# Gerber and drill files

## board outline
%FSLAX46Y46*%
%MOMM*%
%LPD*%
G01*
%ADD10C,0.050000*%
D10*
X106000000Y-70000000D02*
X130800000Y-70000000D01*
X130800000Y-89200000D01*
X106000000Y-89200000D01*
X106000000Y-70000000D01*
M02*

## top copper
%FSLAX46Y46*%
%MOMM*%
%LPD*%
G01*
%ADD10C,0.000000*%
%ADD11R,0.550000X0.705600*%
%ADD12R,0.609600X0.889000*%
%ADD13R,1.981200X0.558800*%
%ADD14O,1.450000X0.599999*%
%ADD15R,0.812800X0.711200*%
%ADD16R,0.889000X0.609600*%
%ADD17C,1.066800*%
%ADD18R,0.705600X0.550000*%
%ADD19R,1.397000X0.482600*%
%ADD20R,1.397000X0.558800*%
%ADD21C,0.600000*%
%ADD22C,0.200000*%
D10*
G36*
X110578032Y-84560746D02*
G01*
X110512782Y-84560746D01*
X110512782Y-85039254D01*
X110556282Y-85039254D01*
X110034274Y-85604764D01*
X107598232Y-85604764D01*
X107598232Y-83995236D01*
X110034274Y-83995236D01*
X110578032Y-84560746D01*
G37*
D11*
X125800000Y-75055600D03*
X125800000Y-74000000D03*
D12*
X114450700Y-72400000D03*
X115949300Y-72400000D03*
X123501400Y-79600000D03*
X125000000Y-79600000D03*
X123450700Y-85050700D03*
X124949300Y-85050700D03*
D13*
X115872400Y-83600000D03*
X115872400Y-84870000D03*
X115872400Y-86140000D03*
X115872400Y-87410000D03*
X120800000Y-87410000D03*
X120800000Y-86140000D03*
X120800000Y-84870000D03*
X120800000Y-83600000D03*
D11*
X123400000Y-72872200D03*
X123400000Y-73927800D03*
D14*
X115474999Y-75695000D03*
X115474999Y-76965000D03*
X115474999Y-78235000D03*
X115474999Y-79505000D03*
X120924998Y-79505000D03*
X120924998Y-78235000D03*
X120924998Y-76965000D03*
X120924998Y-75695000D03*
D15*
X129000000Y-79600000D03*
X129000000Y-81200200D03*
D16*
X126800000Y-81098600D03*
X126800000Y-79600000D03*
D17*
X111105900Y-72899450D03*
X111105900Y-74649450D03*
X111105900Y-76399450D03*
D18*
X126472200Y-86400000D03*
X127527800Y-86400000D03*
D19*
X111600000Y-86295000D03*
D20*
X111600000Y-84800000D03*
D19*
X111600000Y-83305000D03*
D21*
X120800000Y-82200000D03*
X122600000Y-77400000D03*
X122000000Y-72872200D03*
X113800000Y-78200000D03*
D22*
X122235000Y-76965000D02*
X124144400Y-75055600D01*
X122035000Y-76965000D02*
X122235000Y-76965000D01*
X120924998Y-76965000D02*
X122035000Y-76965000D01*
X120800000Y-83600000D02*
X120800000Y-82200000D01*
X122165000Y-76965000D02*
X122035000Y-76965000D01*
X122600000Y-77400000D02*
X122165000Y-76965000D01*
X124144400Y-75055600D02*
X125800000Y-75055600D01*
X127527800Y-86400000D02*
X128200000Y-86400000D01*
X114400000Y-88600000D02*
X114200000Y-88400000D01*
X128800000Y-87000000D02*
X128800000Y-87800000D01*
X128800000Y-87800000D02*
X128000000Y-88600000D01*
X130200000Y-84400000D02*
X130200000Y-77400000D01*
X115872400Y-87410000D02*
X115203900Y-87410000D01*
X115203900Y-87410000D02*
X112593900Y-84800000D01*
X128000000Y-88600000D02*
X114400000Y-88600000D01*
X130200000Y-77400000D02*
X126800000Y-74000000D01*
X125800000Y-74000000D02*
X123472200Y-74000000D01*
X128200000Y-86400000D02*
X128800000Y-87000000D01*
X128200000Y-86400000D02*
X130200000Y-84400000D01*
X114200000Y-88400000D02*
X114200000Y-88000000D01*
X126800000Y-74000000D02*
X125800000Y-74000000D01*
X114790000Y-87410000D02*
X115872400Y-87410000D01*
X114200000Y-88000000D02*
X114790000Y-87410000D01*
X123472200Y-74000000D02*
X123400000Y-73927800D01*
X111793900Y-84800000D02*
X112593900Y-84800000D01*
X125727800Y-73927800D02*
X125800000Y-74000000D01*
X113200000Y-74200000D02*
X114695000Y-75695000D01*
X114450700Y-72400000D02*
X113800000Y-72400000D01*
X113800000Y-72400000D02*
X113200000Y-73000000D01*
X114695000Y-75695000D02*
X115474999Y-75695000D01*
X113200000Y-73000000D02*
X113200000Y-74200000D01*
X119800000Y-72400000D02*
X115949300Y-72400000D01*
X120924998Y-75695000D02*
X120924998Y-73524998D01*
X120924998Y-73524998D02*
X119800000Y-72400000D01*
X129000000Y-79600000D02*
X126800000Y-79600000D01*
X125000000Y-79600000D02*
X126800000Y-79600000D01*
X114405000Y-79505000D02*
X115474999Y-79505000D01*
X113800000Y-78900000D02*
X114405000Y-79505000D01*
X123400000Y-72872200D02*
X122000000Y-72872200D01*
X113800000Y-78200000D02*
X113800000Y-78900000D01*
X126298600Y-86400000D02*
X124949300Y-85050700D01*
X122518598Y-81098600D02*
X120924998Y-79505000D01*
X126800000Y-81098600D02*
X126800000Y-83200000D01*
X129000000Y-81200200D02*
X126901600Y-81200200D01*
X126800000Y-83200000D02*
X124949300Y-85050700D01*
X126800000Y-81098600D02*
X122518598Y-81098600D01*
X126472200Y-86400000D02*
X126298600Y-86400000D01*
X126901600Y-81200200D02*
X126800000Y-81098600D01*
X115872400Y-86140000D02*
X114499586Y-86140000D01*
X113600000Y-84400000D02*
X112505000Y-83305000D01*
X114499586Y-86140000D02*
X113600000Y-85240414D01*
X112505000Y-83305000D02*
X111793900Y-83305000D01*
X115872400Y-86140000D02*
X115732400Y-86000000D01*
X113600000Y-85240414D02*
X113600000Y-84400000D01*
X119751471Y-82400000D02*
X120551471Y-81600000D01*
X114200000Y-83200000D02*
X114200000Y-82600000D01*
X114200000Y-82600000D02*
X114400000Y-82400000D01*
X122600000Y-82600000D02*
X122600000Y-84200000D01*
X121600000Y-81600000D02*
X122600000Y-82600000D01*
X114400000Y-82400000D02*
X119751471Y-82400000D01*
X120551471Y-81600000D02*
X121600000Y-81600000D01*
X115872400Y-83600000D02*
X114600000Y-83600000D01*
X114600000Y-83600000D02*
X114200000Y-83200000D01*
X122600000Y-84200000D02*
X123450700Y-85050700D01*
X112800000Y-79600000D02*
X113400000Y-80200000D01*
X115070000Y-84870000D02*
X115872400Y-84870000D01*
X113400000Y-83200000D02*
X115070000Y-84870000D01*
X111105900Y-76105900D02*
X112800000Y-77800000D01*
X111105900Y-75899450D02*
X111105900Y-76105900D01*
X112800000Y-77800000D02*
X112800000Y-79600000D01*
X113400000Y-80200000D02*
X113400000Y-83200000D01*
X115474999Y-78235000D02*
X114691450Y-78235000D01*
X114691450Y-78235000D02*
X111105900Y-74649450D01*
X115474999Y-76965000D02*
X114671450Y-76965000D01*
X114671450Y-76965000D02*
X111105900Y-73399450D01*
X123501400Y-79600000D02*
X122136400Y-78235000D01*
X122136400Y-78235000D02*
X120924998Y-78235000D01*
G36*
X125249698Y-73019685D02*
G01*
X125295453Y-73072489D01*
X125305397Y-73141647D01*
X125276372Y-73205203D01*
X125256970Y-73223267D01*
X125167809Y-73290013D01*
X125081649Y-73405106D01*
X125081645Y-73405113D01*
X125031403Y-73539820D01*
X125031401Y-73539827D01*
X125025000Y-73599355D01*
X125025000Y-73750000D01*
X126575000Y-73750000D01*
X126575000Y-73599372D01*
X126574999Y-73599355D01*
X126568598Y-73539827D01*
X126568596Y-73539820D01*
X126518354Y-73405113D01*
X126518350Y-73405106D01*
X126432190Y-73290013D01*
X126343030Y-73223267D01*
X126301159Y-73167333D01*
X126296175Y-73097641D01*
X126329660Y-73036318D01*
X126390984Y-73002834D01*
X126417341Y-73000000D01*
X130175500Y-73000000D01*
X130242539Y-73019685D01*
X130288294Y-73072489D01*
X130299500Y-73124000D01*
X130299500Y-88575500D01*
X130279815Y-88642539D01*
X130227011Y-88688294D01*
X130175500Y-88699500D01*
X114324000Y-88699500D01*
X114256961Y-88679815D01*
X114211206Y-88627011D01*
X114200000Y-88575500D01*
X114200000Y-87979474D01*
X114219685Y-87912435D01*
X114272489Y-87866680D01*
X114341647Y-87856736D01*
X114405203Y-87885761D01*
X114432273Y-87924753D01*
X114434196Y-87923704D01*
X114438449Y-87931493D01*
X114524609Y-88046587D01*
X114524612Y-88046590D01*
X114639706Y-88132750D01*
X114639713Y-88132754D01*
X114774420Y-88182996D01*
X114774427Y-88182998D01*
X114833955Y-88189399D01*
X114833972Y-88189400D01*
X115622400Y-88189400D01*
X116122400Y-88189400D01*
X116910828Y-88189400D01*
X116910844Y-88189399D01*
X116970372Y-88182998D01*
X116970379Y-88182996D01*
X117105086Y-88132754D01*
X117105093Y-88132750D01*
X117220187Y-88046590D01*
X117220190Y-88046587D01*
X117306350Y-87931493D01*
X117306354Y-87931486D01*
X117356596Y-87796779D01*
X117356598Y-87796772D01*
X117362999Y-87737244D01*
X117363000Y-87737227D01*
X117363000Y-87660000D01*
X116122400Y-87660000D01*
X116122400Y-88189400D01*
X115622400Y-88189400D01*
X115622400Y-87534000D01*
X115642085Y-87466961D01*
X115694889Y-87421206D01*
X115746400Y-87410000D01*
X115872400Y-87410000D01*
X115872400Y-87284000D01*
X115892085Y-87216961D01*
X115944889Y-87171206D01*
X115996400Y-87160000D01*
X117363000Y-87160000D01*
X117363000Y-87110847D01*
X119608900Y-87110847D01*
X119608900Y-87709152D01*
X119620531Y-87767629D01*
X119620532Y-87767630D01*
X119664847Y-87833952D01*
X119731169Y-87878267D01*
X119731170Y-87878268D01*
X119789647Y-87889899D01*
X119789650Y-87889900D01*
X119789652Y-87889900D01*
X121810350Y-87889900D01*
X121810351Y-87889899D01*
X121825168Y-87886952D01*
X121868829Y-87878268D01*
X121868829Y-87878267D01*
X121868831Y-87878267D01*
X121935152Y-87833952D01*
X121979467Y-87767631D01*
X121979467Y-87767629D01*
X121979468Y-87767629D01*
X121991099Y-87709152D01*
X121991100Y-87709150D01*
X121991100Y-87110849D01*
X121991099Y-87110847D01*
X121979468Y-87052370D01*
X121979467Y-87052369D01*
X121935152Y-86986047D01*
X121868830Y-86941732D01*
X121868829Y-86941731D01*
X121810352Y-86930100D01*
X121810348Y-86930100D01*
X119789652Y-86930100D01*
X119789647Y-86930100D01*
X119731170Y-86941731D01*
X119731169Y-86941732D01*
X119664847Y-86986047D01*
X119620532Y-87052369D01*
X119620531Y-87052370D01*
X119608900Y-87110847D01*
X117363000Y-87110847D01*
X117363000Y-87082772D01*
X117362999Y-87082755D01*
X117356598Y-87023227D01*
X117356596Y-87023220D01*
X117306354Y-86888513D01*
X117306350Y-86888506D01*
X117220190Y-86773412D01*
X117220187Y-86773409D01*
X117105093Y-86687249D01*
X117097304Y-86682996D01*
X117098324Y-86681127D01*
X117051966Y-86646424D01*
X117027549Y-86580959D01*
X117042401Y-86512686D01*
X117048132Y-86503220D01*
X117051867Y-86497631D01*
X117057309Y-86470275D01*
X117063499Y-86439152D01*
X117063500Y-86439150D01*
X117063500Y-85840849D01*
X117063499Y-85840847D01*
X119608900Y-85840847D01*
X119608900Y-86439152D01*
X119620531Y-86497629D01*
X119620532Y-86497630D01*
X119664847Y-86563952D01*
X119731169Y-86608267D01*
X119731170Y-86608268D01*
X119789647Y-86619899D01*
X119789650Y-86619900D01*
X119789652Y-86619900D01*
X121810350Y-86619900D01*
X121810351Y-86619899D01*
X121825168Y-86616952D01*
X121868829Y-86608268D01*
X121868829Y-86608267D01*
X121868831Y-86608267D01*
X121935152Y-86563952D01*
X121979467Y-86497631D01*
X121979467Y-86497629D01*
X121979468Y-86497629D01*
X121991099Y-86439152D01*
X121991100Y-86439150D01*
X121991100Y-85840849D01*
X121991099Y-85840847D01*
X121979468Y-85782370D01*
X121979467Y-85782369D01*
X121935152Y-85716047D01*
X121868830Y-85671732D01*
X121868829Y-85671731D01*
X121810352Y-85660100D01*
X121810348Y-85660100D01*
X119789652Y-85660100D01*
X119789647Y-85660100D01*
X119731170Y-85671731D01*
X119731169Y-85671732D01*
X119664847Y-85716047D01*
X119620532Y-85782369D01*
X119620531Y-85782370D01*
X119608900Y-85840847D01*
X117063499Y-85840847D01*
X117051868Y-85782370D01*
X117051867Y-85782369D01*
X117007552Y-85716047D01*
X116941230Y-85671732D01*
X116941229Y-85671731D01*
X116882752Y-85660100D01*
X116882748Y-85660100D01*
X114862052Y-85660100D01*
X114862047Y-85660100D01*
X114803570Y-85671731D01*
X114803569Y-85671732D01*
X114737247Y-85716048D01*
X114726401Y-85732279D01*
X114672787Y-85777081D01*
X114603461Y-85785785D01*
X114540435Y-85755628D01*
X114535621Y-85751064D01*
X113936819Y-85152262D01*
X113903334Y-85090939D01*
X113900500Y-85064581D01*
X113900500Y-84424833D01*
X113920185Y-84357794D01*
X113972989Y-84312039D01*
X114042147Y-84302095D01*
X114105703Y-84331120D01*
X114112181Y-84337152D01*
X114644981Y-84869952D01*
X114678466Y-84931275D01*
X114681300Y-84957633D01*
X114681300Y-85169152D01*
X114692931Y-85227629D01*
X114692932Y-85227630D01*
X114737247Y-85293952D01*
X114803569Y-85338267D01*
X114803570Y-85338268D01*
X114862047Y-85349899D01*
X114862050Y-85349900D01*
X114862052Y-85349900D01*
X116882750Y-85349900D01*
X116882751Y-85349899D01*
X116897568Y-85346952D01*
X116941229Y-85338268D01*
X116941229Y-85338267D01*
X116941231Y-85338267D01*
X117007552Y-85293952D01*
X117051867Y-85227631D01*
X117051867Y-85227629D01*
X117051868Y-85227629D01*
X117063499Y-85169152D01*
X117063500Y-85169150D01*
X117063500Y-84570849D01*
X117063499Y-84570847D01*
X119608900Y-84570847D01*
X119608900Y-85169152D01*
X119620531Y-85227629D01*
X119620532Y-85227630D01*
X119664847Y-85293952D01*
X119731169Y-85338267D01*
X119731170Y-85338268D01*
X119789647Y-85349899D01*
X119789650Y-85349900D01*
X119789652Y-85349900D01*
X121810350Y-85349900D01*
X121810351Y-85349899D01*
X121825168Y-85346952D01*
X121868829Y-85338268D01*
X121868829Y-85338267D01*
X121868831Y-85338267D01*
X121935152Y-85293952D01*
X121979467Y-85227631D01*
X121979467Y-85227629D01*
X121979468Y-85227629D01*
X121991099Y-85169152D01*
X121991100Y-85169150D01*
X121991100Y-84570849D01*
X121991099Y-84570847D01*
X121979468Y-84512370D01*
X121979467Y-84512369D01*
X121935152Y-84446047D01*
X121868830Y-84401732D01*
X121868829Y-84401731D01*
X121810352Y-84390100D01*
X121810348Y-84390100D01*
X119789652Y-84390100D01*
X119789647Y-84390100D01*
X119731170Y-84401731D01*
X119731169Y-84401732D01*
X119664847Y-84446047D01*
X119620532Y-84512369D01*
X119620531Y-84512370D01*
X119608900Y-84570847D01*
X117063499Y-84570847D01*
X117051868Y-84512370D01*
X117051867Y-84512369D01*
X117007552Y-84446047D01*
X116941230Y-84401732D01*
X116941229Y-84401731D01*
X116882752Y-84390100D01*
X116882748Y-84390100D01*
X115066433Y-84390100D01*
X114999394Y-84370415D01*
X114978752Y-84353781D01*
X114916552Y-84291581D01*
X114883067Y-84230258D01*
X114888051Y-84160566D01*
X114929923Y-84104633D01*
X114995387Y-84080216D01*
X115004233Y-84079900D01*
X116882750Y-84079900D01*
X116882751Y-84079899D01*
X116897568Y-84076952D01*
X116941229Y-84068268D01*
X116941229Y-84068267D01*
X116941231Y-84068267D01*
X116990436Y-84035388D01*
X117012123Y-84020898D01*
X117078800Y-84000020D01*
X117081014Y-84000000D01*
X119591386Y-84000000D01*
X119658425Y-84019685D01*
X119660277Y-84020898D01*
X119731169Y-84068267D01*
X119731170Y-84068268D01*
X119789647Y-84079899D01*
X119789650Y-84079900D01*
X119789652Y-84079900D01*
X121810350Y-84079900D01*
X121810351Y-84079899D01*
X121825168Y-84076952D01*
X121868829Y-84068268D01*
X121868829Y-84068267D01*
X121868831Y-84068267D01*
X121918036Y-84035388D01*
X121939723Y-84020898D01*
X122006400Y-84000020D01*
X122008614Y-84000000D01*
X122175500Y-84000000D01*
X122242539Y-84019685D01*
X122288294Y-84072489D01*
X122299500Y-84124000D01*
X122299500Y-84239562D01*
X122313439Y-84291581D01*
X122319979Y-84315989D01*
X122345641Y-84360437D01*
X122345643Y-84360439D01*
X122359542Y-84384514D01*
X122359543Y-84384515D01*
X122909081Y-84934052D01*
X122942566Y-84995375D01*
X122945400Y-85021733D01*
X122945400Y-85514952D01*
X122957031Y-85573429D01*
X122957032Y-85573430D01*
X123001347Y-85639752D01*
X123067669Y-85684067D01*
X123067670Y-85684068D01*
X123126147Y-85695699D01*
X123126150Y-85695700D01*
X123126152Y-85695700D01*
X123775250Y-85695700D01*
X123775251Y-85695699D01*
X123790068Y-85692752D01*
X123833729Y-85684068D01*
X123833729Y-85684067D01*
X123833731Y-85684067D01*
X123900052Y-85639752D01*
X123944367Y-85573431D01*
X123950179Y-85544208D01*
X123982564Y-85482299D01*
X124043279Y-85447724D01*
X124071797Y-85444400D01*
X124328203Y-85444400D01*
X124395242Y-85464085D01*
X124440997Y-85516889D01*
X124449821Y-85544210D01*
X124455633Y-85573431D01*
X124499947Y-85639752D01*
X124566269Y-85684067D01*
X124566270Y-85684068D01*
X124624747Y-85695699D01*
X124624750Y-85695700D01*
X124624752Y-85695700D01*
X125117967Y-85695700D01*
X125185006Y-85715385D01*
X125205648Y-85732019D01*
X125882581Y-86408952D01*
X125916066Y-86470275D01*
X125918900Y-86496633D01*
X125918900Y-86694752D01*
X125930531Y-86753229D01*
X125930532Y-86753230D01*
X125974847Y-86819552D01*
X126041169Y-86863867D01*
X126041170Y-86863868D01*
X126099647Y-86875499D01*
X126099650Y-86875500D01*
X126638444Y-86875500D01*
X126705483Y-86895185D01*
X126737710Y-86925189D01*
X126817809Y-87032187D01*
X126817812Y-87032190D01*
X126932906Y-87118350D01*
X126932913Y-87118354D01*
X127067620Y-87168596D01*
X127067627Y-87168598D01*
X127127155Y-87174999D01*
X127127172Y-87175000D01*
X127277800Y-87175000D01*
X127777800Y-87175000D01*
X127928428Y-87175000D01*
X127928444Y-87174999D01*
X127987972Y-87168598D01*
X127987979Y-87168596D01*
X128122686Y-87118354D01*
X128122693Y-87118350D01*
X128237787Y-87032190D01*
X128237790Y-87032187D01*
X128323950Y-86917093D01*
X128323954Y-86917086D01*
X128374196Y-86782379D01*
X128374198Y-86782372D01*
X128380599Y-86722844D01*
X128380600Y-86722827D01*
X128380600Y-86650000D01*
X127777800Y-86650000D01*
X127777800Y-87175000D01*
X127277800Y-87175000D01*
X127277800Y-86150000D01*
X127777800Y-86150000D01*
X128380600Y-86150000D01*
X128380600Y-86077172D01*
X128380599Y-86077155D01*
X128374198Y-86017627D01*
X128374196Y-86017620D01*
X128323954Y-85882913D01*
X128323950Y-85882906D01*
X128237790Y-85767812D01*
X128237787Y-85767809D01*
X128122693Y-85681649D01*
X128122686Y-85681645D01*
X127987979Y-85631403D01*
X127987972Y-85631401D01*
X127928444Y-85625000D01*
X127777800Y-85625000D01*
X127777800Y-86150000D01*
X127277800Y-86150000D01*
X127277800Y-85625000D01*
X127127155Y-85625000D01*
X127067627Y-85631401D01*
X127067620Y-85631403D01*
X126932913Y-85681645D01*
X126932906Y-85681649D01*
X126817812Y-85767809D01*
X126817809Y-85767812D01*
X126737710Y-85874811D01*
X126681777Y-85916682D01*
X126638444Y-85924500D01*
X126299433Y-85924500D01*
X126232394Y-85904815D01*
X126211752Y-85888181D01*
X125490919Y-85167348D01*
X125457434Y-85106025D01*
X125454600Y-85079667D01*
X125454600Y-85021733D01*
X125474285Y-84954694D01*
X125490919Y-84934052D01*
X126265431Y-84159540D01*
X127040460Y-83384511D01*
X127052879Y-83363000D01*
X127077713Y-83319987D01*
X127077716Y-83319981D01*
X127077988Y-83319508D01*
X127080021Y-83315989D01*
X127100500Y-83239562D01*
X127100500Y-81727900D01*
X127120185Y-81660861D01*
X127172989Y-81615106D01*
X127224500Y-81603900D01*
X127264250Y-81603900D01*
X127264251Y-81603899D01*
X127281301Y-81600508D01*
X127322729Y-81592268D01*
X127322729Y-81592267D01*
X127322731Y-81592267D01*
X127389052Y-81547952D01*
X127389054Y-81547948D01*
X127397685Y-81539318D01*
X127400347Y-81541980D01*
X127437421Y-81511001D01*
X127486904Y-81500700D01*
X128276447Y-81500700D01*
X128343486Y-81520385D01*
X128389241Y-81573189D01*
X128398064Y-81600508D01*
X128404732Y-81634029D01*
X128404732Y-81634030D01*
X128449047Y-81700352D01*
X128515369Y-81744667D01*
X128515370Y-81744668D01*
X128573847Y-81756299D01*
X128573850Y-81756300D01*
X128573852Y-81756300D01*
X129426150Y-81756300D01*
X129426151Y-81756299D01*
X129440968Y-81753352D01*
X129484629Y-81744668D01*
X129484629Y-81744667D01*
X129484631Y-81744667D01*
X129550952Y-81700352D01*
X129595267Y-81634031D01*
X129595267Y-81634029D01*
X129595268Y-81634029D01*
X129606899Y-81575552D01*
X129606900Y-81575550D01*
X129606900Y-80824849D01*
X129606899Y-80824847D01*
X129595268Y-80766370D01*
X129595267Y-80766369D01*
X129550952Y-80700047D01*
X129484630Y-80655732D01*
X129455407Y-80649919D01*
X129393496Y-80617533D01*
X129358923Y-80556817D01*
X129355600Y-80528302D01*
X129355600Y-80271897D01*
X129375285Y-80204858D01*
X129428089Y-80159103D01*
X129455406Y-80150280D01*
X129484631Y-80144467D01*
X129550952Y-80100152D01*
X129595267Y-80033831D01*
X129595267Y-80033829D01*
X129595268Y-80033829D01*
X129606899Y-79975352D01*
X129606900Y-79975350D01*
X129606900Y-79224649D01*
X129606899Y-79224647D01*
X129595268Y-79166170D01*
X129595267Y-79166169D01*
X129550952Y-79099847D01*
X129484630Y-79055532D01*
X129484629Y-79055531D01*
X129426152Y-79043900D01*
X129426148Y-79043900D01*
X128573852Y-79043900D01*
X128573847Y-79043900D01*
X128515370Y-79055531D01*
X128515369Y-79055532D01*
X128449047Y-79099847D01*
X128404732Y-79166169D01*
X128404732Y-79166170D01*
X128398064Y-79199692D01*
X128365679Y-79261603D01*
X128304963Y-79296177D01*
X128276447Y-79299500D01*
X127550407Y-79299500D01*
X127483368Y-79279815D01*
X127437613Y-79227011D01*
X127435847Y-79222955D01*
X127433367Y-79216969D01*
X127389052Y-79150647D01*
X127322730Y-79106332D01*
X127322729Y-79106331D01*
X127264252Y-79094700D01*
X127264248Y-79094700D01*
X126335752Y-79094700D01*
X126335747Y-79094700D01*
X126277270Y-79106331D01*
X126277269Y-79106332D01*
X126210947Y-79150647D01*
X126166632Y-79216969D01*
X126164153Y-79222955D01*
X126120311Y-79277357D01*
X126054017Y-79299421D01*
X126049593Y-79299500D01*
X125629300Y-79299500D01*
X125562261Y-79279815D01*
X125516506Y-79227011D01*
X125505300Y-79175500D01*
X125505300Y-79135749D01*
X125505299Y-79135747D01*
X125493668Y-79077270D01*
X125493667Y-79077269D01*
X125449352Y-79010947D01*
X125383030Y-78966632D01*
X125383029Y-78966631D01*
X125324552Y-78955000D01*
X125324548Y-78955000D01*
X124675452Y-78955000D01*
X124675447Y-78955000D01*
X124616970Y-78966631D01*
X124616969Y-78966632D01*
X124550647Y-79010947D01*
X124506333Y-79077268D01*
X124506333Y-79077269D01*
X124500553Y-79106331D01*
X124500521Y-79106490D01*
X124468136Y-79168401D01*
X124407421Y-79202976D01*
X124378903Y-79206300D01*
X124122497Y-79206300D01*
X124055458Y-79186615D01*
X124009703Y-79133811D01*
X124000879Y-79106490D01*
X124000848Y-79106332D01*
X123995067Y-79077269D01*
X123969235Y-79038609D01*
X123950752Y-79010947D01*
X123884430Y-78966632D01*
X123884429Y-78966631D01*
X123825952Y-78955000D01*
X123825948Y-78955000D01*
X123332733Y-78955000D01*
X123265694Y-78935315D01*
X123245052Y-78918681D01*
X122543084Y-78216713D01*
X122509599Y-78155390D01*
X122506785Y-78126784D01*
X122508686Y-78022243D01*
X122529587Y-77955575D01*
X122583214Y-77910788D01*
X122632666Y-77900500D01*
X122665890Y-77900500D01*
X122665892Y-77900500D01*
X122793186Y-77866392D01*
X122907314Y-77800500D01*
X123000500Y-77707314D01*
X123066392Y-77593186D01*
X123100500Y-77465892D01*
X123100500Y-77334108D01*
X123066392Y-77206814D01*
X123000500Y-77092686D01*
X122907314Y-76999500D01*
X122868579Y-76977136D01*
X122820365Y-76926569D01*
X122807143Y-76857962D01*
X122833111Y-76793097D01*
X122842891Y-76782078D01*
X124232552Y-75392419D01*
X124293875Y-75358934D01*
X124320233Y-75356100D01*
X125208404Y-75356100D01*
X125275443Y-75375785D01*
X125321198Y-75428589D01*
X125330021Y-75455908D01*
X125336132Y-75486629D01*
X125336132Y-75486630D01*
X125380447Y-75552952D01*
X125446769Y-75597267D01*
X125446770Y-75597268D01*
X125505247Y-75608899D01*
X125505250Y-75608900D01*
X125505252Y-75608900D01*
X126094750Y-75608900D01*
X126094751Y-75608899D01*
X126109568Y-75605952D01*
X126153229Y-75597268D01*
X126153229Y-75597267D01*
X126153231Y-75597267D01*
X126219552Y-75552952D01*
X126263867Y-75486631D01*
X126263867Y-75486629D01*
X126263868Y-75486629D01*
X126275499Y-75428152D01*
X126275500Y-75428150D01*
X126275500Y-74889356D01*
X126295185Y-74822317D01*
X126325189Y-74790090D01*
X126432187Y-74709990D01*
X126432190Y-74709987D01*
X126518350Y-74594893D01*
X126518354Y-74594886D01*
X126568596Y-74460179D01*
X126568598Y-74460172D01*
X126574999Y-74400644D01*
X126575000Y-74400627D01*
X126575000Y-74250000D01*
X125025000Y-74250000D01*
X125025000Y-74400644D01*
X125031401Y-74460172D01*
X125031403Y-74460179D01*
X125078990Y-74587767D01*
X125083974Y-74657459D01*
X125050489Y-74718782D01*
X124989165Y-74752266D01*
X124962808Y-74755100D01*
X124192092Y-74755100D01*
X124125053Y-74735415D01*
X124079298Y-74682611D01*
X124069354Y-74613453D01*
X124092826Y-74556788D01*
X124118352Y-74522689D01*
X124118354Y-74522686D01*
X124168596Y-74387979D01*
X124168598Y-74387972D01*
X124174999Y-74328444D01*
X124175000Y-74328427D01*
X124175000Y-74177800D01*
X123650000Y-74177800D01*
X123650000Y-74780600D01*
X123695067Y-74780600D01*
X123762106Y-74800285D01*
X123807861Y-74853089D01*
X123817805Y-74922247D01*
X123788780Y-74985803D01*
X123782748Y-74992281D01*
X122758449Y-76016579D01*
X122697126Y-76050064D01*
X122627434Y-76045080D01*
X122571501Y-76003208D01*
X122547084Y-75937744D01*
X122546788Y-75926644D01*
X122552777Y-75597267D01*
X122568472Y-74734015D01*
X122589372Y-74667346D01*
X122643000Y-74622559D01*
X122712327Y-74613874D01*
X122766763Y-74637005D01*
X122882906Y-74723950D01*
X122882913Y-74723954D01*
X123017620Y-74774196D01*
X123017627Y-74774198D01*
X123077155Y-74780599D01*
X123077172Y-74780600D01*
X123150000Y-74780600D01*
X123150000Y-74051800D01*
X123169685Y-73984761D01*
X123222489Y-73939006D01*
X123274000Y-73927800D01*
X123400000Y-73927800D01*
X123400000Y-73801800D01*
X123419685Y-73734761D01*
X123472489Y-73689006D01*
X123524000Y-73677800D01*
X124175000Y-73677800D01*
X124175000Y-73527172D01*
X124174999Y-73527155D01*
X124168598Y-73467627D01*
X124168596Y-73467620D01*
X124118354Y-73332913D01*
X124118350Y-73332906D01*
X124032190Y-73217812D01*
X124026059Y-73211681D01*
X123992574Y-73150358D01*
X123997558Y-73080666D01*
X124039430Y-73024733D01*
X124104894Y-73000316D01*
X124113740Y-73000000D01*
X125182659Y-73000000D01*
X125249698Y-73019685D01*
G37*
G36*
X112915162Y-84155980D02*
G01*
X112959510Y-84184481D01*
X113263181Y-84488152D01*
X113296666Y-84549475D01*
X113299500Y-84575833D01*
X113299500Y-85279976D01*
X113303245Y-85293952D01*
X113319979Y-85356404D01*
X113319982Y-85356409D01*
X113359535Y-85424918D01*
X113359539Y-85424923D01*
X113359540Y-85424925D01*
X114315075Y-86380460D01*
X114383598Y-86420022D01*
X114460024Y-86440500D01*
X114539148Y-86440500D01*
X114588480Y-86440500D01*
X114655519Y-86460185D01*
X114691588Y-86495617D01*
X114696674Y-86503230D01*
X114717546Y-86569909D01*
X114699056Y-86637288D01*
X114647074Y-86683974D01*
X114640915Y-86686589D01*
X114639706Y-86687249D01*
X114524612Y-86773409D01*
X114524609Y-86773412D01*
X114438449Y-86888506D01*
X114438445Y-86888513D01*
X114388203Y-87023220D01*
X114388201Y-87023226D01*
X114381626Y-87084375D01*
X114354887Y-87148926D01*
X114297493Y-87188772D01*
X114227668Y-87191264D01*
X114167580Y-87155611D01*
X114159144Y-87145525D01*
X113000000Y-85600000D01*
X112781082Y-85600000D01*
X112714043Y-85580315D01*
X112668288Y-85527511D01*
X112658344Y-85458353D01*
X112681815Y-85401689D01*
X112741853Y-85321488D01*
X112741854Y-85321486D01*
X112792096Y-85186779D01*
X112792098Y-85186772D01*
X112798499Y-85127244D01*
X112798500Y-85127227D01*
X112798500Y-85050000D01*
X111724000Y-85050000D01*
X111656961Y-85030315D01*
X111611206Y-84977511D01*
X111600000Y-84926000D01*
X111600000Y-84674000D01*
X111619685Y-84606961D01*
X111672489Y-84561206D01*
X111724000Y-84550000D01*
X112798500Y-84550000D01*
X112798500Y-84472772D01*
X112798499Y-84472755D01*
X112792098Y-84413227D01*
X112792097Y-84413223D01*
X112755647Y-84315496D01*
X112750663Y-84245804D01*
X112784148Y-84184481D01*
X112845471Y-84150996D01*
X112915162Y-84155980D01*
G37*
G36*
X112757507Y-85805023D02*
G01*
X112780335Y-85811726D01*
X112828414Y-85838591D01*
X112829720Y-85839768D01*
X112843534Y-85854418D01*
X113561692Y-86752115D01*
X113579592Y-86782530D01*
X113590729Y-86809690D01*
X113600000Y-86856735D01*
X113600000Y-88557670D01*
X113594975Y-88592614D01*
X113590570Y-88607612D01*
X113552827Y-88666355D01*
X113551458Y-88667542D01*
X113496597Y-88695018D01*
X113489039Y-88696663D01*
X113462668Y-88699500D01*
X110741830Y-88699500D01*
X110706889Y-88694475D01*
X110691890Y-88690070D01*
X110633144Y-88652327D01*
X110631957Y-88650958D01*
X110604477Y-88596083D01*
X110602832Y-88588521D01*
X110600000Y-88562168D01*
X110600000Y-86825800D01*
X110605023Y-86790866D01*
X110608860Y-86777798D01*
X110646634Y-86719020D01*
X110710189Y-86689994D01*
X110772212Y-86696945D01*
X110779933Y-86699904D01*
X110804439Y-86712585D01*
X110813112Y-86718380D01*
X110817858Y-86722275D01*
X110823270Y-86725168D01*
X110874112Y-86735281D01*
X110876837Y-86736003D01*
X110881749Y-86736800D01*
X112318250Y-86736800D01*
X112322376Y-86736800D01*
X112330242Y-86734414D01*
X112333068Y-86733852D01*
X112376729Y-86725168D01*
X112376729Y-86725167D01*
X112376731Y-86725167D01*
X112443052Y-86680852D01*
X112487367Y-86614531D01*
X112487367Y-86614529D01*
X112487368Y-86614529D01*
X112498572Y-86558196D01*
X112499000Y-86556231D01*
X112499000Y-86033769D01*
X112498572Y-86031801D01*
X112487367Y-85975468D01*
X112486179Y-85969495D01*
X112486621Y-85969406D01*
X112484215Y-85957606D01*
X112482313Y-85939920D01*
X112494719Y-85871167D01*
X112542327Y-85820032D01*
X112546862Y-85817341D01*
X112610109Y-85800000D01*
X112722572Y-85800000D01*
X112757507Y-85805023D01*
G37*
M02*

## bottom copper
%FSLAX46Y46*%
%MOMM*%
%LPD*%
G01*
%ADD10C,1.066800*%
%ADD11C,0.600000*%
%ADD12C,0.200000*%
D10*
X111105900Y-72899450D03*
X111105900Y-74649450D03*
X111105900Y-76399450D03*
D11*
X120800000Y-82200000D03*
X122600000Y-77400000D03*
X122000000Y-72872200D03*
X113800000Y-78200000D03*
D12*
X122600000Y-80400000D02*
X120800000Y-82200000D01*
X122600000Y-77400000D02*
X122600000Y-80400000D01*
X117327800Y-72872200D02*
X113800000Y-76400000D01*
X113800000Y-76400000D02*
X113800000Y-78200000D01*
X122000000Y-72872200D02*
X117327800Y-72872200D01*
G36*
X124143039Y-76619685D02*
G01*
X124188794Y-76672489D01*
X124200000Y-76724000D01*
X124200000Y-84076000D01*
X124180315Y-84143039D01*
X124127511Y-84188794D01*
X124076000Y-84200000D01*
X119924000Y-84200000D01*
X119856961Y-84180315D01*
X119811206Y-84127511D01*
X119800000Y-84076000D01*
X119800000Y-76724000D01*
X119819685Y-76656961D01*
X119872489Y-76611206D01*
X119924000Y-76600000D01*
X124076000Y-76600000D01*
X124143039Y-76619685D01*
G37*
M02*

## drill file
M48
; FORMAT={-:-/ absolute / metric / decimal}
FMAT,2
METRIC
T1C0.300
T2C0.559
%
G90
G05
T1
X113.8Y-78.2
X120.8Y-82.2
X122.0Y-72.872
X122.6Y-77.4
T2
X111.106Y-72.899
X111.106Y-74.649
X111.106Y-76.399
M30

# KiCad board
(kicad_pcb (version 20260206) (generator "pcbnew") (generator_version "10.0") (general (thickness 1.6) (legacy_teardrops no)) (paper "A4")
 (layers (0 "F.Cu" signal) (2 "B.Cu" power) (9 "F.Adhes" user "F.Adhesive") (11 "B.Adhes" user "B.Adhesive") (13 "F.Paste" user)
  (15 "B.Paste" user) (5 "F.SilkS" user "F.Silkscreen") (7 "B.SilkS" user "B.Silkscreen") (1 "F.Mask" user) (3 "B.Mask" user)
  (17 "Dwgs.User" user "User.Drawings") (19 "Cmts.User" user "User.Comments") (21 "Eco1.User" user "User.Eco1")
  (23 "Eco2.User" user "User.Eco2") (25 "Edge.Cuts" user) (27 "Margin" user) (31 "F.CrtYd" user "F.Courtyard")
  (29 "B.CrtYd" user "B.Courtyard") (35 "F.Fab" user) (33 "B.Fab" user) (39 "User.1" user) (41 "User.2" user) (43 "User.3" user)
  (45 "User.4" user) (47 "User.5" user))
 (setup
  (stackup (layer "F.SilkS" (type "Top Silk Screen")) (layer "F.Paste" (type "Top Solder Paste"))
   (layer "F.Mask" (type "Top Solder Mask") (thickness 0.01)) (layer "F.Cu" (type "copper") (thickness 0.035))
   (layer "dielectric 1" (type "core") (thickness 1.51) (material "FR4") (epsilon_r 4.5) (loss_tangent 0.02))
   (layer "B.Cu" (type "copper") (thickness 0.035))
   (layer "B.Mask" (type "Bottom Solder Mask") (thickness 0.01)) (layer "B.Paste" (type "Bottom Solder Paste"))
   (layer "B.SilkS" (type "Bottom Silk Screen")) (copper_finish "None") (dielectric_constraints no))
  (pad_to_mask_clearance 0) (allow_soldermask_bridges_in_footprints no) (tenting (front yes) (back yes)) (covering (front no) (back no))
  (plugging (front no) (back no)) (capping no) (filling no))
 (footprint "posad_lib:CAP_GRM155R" (layer "F.Cu") (at 125.8 74.5278 90)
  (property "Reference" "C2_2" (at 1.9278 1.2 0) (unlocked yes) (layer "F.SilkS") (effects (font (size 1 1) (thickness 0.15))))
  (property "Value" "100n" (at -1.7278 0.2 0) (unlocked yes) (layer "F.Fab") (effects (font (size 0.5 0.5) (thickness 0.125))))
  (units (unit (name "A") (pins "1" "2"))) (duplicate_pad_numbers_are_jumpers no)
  (pad "1" smd rect (at -0.5278 0 90) (size 0.7056 0.55) (layers "F.Cu" "F.Mask" "F.Paste") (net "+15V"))
  (pad "2" smd rect (at 0.5278 0 90) (size 0.7056 0.55) (layers "F.Cu" "F.Mask" "F.Paste") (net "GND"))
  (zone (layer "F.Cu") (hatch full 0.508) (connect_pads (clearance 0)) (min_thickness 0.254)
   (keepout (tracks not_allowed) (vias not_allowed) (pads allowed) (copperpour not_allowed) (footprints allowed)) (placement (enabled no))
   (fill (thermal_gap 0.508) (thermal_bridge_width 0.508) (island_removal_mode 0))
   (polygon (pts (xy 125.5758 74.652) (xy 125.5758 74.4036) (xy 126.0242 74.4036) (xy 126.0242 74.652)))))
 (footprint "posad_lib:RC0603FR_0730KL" (layer "F.Cu") (at 115.2 72.4)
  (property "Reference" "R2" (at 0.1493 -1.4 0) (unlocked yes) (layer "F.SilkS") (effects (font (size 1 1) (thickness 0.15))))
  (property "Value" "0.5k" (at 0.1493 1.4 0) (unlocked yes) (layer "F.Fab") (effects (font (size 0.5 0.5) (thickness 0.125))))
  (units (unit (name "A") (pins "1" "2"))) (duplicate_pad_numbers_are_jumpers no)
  (pad "1" smd rect (at -0.7493 0) (size 0.6096 0.889) (layers "F.Cu" "F.Mask" "F.Paste") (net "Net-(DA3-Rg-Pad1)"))
  (pad "2" smd rect (at 0.7493 0) (size 0.6096 0.889) (layers "F.Cu" "F.Mask" "F.Paste") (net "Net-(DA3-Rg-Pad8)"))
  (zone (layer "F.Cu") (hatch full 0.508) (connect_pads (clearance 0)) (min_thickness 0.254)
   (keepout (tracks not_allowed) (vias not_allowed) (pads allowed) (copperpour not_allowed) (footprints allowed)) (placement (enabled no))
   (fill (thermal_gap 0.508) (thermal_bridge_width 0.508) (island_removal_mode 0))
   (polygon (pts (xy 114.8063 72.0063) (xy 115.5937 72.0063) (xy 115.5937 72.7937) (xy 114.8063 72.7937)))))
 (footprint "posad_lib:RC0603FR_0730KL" (layer "F.Cu") (at 124.2507 79.6)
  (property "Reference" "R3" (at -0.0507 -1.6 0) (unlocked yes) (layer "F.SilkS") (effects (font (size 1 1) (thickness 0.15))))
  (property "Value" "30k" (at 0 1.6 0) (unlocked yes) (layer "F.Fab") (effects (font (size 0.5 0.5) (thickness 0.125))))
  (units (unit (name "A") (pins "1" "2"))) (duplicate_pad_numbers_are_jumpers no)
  (pad "1" smd rect (at -0.7493 0) (size 0.6096 0.889) (layers "F.Cu" "F.Mask" "F.Paste") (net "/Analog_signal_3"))
  (pad "2" smd rect (at 0.7493 0) (size 0.6096 0.889) (layers "F.Cu" "F.Mask" "F.Paste") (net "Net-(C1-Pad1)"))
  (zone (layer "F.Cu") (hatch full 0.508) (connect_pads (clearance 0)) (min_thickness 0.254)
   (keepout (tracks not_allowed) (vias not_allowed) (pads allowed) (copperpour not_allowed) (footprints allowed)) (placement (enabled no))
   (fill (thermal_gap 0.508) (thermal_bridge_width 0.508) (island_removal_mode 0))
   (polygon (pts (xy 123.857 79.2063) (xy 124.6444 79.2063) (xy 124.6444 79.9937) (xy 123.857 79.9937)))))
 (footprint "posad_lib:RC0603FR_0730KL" (layer "F.Cu") (at 124.2 85.0507)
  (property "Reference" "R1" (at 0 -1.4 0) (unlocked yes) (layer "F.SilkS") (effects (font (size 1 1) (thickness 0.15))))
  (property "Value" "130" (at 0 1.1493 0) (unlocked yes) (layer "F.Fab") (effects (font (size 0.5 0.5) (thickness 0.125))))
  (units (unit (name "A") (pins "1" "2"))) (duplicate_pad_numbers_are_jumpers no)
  (pad "1" smd rect (at -0.7493 0) (size 0.6096 0.889) (layers "F.Cu" "F.Mask" "F.Paste") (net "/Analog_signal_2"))
  (pad "2" smd rect (at 0.7493 0) (size 0.6096 0.889) (layers "F.Cu" "F.Mask" "F.Paste") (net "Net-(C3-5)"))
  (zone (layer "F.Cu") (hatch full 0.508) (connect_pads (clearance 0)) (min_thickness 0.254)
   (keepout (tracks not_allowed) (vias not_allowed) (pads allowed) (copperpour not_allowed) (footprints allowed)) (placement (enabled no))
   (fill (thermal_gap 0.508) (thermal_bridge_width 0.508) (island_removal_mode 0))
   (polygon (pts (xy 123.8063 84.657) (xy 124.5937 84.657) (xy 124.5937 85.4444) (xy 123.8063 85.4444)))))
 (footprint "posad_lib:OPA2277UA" (layer "F.Cu") (at 118.3362 85.505)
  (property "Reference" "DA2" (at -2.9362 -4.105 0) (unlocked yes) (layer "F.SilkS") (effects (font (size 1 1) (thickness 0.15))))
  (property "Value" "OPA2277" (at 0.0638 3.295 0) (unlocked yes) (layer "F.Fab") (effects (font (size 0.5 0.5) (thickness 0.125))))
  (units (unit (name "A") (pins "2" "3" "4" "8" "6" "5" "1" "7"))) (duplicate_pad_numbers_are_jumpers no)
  (pad "1" smd rect (at -2.4638 -1.905) (size 1.9812 0.5588) (layers "F.Cu" "F.Mask" "F.Paste") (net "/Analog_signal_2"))
  (pad "2" smd rect (at -2.4638 -0.635) (size 1.9812 0.5588) (layers "F.Cu" "F.Mask" "F.Paste") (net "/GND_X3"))
  (pad "3" smd rect (at -2.4638 0.635) (size 1.9812 0.5588) (layers "F.Cu" "F.Mask" "F.Paste") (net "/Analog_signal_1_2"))
  (pad "4" smd rect (at -2.4638 1.905) (size 1.9812 0.5588) (layers "F.Cu" "F.Mask" "F.Paste") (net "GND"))
  (pad "5" smd rect (at 2.4638 1.905) (size 1.9812 0.5588) (layers "F.Cu" "F.Mask" "F.Paste") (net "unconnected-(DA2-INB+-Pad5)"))
  (pad "6" smd rect (at 2.4638 0.635) (size 1.9812 0.5588) (layers "F.Cu" "F.Mask" "F.Paste") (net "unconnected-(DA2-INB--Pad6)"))
  (pad "7" smd rect (at 2.4638 -0.635) (size 1.9812 0.5588) (layers "F.Cu" "F.Mask" "F.Paste") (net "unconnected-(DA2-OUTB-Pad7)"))
  (pad "8" smd rect (at 2.4638 -1.905) (size 1.9812 0.5588) (layers "F.Cu" "F.Mask" "F.Paste") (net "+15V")))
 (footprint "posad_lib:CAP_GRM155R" (layer "F.Cu") (at 123.4 73.4 -90)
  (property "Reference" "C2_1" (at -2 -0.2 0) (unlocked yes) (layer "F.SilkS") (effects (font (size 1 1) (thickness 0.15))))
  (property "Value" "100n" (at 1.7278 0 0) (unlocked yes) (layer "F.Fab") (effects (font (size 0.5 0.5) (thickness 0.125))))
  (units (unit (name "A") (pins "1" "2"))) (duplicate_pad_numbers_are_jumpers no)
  (pad "1" smd rect (at -0.5278 0 270) (size 0.7056 0.55) (layers "F.Cu" "F.Mask" "F.Paste") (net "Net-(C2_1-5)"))
  (pad "2" smd rect (at 0.5278 0 270) (size 0.7056 0.55) (layers "F.Cu" "F.Mask" "F.Paste") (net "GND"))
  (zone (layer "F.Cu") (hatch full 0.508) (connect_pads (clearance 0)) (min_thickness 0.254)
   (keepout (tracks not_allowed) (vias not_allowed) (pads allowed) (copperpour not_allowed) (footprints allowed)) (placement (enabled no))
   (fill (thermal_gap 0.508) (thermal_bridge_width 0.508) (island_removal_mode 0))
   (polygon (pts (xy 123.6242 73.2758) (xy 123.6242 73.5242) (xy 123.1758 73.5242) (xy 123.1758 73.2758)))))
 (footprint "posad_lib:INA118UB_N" (layer "F.Cu") (at 118.2 77.6)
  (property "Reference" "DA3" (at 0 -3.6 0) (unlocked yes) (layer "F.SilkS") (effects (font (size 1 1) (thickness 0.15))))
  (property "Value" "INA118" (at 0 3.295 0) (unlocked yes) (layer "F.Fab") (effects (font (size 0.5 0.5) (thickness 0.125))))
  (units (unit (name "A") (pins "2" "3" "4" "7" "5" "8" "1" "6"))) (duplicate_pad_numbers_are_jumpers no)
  (pad "1" smd oval (at -2.725001 -1.905 90) (size 0.599999 1.45) (layers "F.Cu" "F.Mask" "F.Paste") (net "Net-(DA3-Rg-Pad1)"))
  (pad "2" smd oval (at -2.725001 -0.635 90) (size 0.599999 1.45) (layers "F.Cu" "F.Mask" "F.Paste") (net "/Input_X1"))
  (pad "3" smd oval (at -2.725001 0.635 90) (size 0.599999 1.45) (layers "F.Cu" "F.Mask" "F.Paste") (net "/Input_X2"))
  (pad "4" smd oval (at -2.725001 1.905 90) (size 0.599999 1.45) (layers "F.Cu" "F.Mask" "F.Paste") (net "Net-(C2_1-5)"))
  (pad "5" smd oval (at 2.724998 1.905 90) (size 0.599999 1.45) (layers "F.Cu" "F.Mask" "F.Paste") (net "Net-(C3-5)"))
  (pad "6" smd oval (at 2.724998 0.635 90) (size 0.599999 1.45) (layers "F.Cu" "F.Mask" "F.Paste") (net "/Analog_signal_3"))
  (pad "7" smd oval (at 2.724998 -0.635 90) (size 0.599999 1.45) (layers "F.Cu" "F.Mask" "F.Paste") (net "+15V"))
  (pad "8" smd oval (at 2.724998 -1.905 90) (size 0.599999 1.45) (layers "F.Cu" "F.Mask" "F.Paste") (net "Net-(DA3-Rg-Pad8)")))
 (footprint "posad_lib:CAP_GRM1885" (layer "F.Cu") (at 129 80.4001 -90)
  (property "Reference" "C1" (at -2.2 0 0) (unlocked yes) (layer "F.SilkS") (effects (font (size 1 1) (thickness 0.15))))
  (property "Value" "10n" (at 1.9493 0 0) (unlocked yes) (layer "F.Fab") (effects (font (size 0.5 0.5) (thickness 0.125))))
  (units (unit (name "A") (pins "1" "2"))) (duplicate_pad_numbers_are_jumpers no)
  (pad "1" smd rect (at -0.8001 0 270) (size 0.7112 0.8128) (layers "F.Cu" "F.Mask" "F.Paste") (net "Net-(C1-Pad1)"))
  (pad "2" smd rect (at 0.8001 0 270) (size 0.7112 0.8128) (layers "F.Cu" "F.Mask" "F.Paste") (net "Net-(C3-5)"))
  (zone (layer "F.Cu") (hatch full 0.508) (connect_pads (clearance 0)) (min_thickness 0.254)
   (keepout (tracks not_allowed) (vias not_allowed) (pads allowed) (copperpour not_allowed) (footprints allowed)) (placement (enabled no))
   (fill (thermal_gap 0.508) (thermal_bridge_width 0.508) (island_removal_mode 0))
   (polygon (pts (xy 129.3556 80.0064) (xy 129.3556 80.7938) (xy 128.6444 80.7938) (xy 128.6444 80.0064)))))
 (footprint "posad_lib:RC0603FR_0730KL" (layer "F.Cu") (at 126.8 80.3493 90)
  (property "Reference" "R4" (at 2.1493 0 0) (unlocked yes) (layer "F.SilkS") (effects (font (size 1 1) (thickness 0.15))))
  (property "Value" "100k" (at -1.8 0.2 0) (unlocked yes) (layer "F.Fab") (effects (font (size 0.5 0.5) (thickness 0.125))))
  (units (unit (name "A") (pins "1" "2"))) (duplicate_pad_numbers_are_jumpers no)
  (pad "1" smd rect (at -0.7493 0 90) (size 0.6096 0.889) (layers "F.Cu" "F.Mask" "F.Paste") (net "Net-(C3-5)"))
  (pad "2" smd rect (at 0.7493 0 90) (size 0.6096 0.889) (layers "F.Cu" "F.Mask" "F.Paste") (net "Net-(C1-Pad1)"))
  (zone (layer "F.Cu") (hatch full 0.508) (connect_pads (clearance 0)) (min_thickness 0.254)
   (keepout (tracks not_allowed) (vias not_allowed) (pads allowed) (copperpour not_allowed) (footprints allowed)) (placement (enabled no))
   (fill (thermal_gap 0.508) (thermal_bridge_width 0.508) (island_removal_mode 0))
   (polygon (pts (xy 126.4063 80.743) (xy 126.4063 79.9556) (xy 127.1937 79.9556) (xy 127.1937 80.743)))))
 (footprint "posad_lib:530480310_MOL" (layer "F.Cu") (at 111.1059 73.39945 -90)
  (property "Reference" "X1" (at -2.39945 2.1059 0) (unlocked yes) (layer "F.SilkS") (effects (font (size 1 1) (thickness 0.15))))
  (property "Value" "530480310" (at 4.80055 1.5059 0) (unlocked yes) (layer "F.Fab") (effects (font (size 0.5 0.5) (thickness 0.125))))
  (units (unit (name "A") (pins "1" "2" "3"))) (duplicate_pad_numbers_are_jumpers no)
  (pad "1" thru_hole circle (at -0.5 0 270) (size 1.0668 1.0668) (drill 0.5588) (layers "*.Cu" "*.Mask") (remove_unused_layers no)
   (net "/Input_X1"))
  (pad "2" thru_hole circle (at 1.25 0 270) (size 1.0668 1.0668) (drill 0.5588) (layers "*.Cu" "*.Mask") (remove_unused_layers no)
   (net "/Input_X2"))
  (pad "3" thru_hole circle (at 3 0 270) (size 1.0668 1.0668) (drill 0.5588) (layers "*.Cu" "*.Mask") (remove_unused_layers no)
   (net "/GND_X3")))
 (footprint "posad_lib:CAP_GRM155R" (layer "F.Cu") (at 127 86.4)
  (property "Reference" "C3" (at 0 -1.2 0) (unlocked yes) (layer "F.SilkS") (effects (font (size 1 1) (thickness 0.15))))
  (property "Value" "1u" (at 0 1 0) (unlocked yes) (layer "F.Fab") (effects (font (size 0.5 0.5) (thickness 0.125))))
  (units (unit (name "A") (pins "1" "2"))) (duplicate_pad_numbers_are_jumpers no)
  (pad "1" smd rect (at -0.5278 0) (size 0.7056 0.55) (layers "F.Cu" "F.Mask" "F.Paste") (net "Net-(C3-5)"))
  (pad "2" smd rect (at 0.5278 0) (size 0.7056 0.55) (layers "F.Cu" "F.Mask" "F.Paste") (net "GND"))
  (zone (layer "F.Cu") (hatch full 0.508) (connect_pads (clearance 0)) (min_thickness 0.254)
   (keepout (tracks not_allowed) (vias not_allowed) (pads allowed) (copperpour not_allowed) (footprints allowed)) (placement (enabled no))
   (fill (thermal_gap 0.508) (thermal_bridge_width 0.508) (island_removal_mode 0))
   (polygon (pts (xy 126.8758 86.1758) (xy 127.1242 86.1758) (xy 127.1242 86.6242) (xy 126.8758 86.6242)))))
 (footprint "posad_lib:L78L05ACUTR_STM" (layer "F.Cu") (at 109.6061 84.8 90)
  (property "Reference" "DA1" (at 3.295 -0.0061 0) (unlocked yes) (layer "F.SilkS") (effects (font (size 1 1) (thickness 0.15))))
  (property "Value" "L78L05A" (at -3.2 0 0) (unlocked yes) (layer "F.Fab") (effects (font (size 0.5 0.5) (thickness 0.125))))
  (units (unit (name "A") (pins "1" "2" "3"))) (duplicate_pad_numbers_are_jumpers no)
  (fp_poly
   (pts (xy -0.239254 0.906682) (xy -0.239254 0.950182) (xy -0.804764 0.428174) (xy -0.804764 -2.007868) (xy 0.804764 -2.007868)
    (xy 0.804764 0.428174) (xy 0.239254 0.971932) (xy 0.239254 0.906682))
   (stroke (width 0) (type solid)) (fill yes) (layer "F.Cu"))
  (pad "1" smd rect (at -1.495 1.9939 90) (size 0.4826 1.397) (layers "F.Cu" "F.Mask" "F.Paste") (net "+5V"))
  (pad "2" smd rect (at 0 1.9939 90) (size 0.5588 1.397) (layers "F.Cu" "F.Mask" "F.Paste") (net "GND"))
  (pad "3" smd rect (at 1.495 1.9939 90) (size 0.4826 1.397) (layers "F.Cu" "F.Mask" "F.Paste") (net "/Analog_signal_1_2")))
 (gr_rect (start 106 70) (end 130.8 89.2) (stroke (width 0.05) (type default)) (fill no) (layer "Edge.Cuts"))
 (segment (start 122.235 76.965) (end 124.1444 75.0556) (width 0.2) (layer "F.Cu") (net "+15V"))
 (segment (start 122.035 76.965) (end 122.235 76.965) (width 0.2) (layer "F.Cu") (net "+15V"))
 (segment (start 120.924998 76.965) (end 122.035 76.965) (width 0.2) (layer "F.Cu") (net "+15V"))
 (segment (start 120.8 83.6) (end 120.8 82.2) (width 0.2) (layer "F.Cu") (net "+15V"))
 (segment (start 122.165 76.965) (end 122.035 76.965) (width 0.2) (layer "F.Cu") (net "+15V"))
 (segment (start 122.6 77.4) (end 122.165 76.965) (width 0.2) (layer "F.Cu") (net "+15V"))
 (segment (start 124.1444 75.0556) (end 125.8 75.0556) (width 0.2) (layer "F.Cu") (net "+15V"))
 (via (at 120.8 82.2) (size 0.6) (drill 0.3) (layers "F.Cu" "B.Cu") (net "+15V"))
 (via (at 122.6 77.4) (size 0.6) (drill 0.3) (layers "F.Cu" "B.Cu") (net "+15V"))
 (segment (start 122.6 80.4) (end 120.8 82.2) (width 0.2) (layer "B.Cu") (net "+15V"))
 (segment (start 122.6 77.4) (end 122.6 80.4) (width 0.2) (layer "B.Cu") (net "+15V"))
 (segment (start 127.5278 86.4) (end 128.2 86.4) (width 0.2) (layer "F.Cu") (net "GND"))
 (segment (start 114.4 88.6) (end 114.2 88.4) (width 0.2) (layer "F.Cu") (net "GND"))
 (segment (start 128.8 87) (end 128.8 87.8) (width 0.2) (layer "F.Cu") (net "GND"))
 (segment (start 128.8 87.8) (end 128 88.6) (width 0.2) (layer "F.Cu") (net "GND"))
 (segment (start 130.2 84.4) (end 130.2 77.4) (width 0.2) (layer "F.Cu") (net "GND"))
 (segment (start 115.8724 87.41) (end 115.2039 87.41) (width 0.2) (layer "F.Cu") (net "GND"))
 (segment (start 115.2039 87.41) (end 112.5939 84.8) (width 0.2) (layer "F.Cu") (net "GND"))
 (segment (start 128 88.6) (end 114.4 88.6) (width 0.2) (layer "F.Cu") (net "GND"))
 (segment (start 130.2 77.4) (end 126.8 74) (width 0.2) (layer "F.Cu") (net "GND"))
 (segment (start 125.8 74) (end 123.4722 74) (width 0.2) (layer "F.Cu") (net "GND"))
 (segment (start 128.2 86.4) (end 128.8 87) (width 0.2) (layer "F.Cu") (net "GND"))
 (segment (start 128.2 86.4) (end 130.2 84.4) (width 0.2) (layer "F.Cu") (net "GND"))
 (segment (start 114.2 88.4) (end 114.2 88) (width 0.2) (layer "F.Cu") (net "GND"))
 (segment (start 126.8 74) (end 125.8 74) (width 0.2) (layer "F.Cu") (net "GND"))
 (segment (start 114.79 87.41) (end 115.8724 87.41) (width 0.2) (layer "F.Cu") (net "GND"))
 (segment (start 114.2 88) (end 114.79 87.41) (width 0.2) (layer "F.Cu") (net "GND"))
 (segment (start 123.4722 74) (end 123.4 73.9278) (width 0.2) (layer "F.Cu") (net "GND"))
 (segment (start 111.7939 84.8) (end 112.5939 84.8) (width 0.2) (layer "F.Cu") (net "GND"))
 (segment (start 125.7278 73.9278) (end 125.8 74) (width 0.2) (layer "F.Cu") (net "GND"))
 (segment (start 113.2 74.2) (end 114.695 75.695) (width 0.2) (layer "F.Cu") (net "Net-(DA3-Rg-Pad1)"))
 (segment (start 114.4507 72.4) (end 113.8 72.4) (width 0.2) (layer "F.Cu") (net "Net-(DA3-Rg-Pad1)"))
 (segment (start 113.8 72.4) (end 113.2 73) (width 0.2) (layer "F.Cu") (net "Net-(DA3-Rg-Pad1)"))
 (segment (start 114.695 75.695) (end 115.474999 75.695) (width 0.2) (layer "F.Cu") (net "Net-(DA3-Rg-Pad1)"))
 (segment (start 113.2 73) (end 113.2 74.2) (width 0.2) (layer "F.Cu") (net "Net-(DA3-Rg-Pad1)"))
 (segment (start 119.8 72.4) (end 115.9493 72.4) (width 0.2) (layer "F.Cu") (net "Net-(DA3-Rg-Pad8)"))
 (segment (start 120.924998 75.695) (end 120.924998 73.524998) (width 0.2) (layer "F.Cu") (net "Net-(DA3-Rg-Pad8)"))
 (segment (start 120.924998 73.524998) (end 119.8 72.4) (width 0.2) (layer "F.Cu") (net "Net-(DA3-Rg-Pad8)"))
 (segment (start 129 79.6) (end 126.8 79.6) (width 0.2) (layer "F.Cu") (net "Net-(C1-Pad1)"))
 (segment (start 125 79.6) (end 126.8 79.6) (width 0.2) (layer "F.Cu") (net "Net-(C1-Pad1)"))
 (segment (start 114.405 79.505) (end 115.474999 79.505) (width 0.2) (layer "F.Cu") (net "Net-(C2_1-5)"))
 (segment (start 113.8 78.9) (end 114.405 79.505) (width 0.2) (layer "F.Cu") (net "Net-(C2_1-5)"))
 (segment (start 123.4 72.8722) (end 122 72.8722) (width 0.2) (layer "F.Cu") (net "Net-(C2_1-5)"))
 (segment (start 113.8 78.2) (end 113.8 78.9) (width 0.2) (layer "F.Cu") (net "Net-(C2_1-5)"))
 (via (at 122 72.8722) (size 0.6) (drill 0.3) (layers "F.Cu" "B.Cu") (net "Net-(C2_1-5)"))
 (via (at 113.8 78.2) (size 0.6) (drill 0.3) (layers "F.Cu" "B.Cu") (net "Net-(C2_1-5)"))
 (segment (start 117.3278 72.8722) (end 113.8 76.4) (width 0.2) (layer "B.Cu") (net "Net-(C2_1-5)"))
 (segment (start 113.8 76.4) (end 113.8 78.2) (width 0.2) (layer "B.Cu") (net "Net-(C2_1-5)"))
 (segment (start 122 72.8722) (end 117.3278 72.8722) (width 0.2) (layer "B.Cu") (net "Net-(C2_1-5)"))
 (segment (start 126.2986 86.4) (end 124.9493 85.0507) (width 0.2) (layer "F.Cu") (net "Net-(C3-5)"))
 (segment (start 122.518598 81.0986) (end 120.924998 79.505) (width 0.2) (layer "F.Cu") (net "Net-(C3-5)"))
 (segment (start 126.8 81.0986) (end 126.8 83.2) (width 0.2) (layer "F.Cu") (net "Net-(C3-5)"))
 (segment (start 129 81.2002) (end 126.9016 81.2002) (width 0.2) (layer "F.Cu") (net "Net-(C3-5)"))
 (segment (start 126.8 83.2) (end 124.9493 85.0507) (width 0.2) (layer "F.Cu") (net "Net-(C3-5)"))
 (segment (start 126.8 81.0986) (end 122.518598 81.0986) (width 0.2) (layer "F.Cu") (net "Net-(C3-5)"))
 (segment (start 126.4722 86.4) (end 126.2986 86.4) (width 0.2) (layer "F.Cu") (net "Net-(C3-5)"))
 (segment (start 126.9016 81.2002) (end 126.8 81.0986) (width 0.2) (layer "F.Cu") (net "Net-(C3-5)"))
 (segment (start 115.8724 86.14) (end 114.499586 86.14) (width 0.2) (layer "F.Cu") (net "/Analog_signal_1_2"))
 (segment (start 113.6 84.4) (end 112.505 83.305) (width 0.2) (layer "F.Cu") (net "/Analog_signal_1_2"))
 (segment (start 114.499586 86.14) (end 113.6 85.240414) (width 0.2) (layer "F.Cu") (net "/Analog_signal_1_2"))
 (segment (start 112.505 83.305) (end 111.7939 83.305) (width 0.2) (layer "F.Cu") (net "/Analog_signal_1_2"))
 (segment (start 115.8724 86.14) (end 115.7324 86) (width 0.2) (layer "F.Cu") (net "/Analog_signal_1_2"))
 (segment (start 113.6 85.240414) (end 113.6 84.4) (width 0.2) (layer "F.Cu") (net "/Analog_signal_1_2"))
 (segment (start 119.751471 82.4) (end 120.551471 81.6) (width 0.2) (layer "F.Cu") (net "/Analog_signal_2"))
 (segment (start 114.2 83.2) (end 114.2 82.6) (width 0.2) (layer "F.Cu") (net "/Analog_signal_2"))
 (segment (start 114.2 82.6) (end 114.4 82.4) (width 0.2) (layer "F.Cu") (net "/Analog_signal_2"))
 (segment (start 122.6 82.6) (end 122.6 84.2) (width 0.2) (layer "F.Cu") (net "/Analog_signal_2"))
 (segment (start 121.6 81.6) (end 122.6 82.6) (width 0.2) (layer "F.Cu") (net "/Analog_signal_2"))
 (segment (start 114.4 82.4) (end 119.751471 82.4) (width 0.2) (layer "F.Cu") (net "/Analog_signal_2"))
 (segment (start 120.551471 81.6) (end 121.6 81.6) (width 0.2) (layer "F.Cu") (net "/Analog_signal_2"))
 (segment (start 115.8724 83.6) (end 114.6 83.6) (width 0.2) (layer "F.Cu") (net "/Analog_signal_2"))
 (segment (start 114.6 83.6) (end 114.2 83.2) (width 0.2) (layer "F.Cu") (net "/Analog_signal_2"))
 (segment (start 122.6 84.2) (end 123.4507 85.0507) (width 0.2) (layer "F.Cu") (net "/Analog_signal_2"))
 (segment (start 112.8 79.6) (end 113.4 80.2) (width 0.2) (layer "F.Cu") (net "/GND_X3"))
 (segment (start 115.07 84.87) (end 115.8724 84.87) (width 0.2) (layer "F.Cu") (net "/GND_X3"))
 (segment (start 113.4 83.2) (end 115.07 84.87) (width 0.2) (layer "F.Cu") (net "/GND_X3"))
 (segment (start 111.1059 76.1059) (end 112.8 77.8) (width 0.2) (layer "F.Cu") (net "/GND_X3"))
 (segment (start 111.1059 75.89945) (end 111.1059 76.1059) (width 0.2) (layer "F.Cu") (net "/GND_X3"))
 (segment (start 112.8 77.8) (end 112.8 79.6) (width 0.2) (layer "F.Cu") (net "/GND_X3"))
 (segment (start 113.4 80.2) (end 113.4 83.2) (width 0.2) (layer "F.Cu") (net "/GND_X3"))
 (segment (start 115.474999 78.235) (end 114.69145 78.235) (width 0.2) (layer "F.Cu") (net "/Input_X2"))
 (segment (start 114.69145 78.235) (end 111.1059 74.64945) (width 0.2) (layer "F.Cu") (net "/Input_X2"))
 (segment (start 115.474999 76.965) (end 114.67145 76.965) (width 0.2) (layer "F.Cu") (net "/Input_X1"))
 (segment (start 114.67145 76.965) (end 111.1059 73.39945) (width 0.2) (layer "F.Cu") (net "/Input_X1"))
 (segment (start 123.5014 79.6) (end 122.1364 78.235) (width 0.2) (layer "F.Cu") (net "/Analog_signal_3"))
 (segment (start 122.1364 78.235) (end 120.924998 78.235) (width 0.2) (layer "F.Cu") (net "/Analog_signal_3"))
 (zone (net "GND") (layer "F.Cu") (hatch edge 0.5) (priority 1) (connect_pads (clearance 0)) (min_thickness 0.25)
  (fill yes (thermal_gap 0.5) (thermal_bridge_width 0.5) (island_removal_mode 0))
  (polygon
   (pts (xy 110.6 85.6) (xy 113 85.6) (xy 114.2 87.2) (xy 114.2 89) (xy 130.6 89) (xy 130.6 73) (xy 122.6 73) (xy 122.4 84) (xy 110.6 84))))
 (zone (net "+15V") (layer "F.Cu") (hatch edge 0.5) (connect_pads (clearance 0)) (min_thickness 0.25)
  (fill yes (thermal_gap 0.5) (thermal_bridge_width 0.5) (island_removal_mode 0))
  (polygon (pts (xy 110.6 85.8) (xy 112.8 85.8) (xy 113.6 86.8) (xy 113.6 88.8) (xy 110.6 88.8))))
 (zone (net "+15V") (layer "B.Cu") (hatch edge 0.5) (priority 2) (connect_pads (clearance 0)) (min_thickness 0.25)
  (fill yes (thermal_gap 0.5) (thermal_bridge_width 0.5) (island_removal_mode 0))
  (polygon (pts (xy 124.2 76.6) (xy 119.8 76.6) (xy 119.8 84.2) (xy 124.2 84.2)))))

